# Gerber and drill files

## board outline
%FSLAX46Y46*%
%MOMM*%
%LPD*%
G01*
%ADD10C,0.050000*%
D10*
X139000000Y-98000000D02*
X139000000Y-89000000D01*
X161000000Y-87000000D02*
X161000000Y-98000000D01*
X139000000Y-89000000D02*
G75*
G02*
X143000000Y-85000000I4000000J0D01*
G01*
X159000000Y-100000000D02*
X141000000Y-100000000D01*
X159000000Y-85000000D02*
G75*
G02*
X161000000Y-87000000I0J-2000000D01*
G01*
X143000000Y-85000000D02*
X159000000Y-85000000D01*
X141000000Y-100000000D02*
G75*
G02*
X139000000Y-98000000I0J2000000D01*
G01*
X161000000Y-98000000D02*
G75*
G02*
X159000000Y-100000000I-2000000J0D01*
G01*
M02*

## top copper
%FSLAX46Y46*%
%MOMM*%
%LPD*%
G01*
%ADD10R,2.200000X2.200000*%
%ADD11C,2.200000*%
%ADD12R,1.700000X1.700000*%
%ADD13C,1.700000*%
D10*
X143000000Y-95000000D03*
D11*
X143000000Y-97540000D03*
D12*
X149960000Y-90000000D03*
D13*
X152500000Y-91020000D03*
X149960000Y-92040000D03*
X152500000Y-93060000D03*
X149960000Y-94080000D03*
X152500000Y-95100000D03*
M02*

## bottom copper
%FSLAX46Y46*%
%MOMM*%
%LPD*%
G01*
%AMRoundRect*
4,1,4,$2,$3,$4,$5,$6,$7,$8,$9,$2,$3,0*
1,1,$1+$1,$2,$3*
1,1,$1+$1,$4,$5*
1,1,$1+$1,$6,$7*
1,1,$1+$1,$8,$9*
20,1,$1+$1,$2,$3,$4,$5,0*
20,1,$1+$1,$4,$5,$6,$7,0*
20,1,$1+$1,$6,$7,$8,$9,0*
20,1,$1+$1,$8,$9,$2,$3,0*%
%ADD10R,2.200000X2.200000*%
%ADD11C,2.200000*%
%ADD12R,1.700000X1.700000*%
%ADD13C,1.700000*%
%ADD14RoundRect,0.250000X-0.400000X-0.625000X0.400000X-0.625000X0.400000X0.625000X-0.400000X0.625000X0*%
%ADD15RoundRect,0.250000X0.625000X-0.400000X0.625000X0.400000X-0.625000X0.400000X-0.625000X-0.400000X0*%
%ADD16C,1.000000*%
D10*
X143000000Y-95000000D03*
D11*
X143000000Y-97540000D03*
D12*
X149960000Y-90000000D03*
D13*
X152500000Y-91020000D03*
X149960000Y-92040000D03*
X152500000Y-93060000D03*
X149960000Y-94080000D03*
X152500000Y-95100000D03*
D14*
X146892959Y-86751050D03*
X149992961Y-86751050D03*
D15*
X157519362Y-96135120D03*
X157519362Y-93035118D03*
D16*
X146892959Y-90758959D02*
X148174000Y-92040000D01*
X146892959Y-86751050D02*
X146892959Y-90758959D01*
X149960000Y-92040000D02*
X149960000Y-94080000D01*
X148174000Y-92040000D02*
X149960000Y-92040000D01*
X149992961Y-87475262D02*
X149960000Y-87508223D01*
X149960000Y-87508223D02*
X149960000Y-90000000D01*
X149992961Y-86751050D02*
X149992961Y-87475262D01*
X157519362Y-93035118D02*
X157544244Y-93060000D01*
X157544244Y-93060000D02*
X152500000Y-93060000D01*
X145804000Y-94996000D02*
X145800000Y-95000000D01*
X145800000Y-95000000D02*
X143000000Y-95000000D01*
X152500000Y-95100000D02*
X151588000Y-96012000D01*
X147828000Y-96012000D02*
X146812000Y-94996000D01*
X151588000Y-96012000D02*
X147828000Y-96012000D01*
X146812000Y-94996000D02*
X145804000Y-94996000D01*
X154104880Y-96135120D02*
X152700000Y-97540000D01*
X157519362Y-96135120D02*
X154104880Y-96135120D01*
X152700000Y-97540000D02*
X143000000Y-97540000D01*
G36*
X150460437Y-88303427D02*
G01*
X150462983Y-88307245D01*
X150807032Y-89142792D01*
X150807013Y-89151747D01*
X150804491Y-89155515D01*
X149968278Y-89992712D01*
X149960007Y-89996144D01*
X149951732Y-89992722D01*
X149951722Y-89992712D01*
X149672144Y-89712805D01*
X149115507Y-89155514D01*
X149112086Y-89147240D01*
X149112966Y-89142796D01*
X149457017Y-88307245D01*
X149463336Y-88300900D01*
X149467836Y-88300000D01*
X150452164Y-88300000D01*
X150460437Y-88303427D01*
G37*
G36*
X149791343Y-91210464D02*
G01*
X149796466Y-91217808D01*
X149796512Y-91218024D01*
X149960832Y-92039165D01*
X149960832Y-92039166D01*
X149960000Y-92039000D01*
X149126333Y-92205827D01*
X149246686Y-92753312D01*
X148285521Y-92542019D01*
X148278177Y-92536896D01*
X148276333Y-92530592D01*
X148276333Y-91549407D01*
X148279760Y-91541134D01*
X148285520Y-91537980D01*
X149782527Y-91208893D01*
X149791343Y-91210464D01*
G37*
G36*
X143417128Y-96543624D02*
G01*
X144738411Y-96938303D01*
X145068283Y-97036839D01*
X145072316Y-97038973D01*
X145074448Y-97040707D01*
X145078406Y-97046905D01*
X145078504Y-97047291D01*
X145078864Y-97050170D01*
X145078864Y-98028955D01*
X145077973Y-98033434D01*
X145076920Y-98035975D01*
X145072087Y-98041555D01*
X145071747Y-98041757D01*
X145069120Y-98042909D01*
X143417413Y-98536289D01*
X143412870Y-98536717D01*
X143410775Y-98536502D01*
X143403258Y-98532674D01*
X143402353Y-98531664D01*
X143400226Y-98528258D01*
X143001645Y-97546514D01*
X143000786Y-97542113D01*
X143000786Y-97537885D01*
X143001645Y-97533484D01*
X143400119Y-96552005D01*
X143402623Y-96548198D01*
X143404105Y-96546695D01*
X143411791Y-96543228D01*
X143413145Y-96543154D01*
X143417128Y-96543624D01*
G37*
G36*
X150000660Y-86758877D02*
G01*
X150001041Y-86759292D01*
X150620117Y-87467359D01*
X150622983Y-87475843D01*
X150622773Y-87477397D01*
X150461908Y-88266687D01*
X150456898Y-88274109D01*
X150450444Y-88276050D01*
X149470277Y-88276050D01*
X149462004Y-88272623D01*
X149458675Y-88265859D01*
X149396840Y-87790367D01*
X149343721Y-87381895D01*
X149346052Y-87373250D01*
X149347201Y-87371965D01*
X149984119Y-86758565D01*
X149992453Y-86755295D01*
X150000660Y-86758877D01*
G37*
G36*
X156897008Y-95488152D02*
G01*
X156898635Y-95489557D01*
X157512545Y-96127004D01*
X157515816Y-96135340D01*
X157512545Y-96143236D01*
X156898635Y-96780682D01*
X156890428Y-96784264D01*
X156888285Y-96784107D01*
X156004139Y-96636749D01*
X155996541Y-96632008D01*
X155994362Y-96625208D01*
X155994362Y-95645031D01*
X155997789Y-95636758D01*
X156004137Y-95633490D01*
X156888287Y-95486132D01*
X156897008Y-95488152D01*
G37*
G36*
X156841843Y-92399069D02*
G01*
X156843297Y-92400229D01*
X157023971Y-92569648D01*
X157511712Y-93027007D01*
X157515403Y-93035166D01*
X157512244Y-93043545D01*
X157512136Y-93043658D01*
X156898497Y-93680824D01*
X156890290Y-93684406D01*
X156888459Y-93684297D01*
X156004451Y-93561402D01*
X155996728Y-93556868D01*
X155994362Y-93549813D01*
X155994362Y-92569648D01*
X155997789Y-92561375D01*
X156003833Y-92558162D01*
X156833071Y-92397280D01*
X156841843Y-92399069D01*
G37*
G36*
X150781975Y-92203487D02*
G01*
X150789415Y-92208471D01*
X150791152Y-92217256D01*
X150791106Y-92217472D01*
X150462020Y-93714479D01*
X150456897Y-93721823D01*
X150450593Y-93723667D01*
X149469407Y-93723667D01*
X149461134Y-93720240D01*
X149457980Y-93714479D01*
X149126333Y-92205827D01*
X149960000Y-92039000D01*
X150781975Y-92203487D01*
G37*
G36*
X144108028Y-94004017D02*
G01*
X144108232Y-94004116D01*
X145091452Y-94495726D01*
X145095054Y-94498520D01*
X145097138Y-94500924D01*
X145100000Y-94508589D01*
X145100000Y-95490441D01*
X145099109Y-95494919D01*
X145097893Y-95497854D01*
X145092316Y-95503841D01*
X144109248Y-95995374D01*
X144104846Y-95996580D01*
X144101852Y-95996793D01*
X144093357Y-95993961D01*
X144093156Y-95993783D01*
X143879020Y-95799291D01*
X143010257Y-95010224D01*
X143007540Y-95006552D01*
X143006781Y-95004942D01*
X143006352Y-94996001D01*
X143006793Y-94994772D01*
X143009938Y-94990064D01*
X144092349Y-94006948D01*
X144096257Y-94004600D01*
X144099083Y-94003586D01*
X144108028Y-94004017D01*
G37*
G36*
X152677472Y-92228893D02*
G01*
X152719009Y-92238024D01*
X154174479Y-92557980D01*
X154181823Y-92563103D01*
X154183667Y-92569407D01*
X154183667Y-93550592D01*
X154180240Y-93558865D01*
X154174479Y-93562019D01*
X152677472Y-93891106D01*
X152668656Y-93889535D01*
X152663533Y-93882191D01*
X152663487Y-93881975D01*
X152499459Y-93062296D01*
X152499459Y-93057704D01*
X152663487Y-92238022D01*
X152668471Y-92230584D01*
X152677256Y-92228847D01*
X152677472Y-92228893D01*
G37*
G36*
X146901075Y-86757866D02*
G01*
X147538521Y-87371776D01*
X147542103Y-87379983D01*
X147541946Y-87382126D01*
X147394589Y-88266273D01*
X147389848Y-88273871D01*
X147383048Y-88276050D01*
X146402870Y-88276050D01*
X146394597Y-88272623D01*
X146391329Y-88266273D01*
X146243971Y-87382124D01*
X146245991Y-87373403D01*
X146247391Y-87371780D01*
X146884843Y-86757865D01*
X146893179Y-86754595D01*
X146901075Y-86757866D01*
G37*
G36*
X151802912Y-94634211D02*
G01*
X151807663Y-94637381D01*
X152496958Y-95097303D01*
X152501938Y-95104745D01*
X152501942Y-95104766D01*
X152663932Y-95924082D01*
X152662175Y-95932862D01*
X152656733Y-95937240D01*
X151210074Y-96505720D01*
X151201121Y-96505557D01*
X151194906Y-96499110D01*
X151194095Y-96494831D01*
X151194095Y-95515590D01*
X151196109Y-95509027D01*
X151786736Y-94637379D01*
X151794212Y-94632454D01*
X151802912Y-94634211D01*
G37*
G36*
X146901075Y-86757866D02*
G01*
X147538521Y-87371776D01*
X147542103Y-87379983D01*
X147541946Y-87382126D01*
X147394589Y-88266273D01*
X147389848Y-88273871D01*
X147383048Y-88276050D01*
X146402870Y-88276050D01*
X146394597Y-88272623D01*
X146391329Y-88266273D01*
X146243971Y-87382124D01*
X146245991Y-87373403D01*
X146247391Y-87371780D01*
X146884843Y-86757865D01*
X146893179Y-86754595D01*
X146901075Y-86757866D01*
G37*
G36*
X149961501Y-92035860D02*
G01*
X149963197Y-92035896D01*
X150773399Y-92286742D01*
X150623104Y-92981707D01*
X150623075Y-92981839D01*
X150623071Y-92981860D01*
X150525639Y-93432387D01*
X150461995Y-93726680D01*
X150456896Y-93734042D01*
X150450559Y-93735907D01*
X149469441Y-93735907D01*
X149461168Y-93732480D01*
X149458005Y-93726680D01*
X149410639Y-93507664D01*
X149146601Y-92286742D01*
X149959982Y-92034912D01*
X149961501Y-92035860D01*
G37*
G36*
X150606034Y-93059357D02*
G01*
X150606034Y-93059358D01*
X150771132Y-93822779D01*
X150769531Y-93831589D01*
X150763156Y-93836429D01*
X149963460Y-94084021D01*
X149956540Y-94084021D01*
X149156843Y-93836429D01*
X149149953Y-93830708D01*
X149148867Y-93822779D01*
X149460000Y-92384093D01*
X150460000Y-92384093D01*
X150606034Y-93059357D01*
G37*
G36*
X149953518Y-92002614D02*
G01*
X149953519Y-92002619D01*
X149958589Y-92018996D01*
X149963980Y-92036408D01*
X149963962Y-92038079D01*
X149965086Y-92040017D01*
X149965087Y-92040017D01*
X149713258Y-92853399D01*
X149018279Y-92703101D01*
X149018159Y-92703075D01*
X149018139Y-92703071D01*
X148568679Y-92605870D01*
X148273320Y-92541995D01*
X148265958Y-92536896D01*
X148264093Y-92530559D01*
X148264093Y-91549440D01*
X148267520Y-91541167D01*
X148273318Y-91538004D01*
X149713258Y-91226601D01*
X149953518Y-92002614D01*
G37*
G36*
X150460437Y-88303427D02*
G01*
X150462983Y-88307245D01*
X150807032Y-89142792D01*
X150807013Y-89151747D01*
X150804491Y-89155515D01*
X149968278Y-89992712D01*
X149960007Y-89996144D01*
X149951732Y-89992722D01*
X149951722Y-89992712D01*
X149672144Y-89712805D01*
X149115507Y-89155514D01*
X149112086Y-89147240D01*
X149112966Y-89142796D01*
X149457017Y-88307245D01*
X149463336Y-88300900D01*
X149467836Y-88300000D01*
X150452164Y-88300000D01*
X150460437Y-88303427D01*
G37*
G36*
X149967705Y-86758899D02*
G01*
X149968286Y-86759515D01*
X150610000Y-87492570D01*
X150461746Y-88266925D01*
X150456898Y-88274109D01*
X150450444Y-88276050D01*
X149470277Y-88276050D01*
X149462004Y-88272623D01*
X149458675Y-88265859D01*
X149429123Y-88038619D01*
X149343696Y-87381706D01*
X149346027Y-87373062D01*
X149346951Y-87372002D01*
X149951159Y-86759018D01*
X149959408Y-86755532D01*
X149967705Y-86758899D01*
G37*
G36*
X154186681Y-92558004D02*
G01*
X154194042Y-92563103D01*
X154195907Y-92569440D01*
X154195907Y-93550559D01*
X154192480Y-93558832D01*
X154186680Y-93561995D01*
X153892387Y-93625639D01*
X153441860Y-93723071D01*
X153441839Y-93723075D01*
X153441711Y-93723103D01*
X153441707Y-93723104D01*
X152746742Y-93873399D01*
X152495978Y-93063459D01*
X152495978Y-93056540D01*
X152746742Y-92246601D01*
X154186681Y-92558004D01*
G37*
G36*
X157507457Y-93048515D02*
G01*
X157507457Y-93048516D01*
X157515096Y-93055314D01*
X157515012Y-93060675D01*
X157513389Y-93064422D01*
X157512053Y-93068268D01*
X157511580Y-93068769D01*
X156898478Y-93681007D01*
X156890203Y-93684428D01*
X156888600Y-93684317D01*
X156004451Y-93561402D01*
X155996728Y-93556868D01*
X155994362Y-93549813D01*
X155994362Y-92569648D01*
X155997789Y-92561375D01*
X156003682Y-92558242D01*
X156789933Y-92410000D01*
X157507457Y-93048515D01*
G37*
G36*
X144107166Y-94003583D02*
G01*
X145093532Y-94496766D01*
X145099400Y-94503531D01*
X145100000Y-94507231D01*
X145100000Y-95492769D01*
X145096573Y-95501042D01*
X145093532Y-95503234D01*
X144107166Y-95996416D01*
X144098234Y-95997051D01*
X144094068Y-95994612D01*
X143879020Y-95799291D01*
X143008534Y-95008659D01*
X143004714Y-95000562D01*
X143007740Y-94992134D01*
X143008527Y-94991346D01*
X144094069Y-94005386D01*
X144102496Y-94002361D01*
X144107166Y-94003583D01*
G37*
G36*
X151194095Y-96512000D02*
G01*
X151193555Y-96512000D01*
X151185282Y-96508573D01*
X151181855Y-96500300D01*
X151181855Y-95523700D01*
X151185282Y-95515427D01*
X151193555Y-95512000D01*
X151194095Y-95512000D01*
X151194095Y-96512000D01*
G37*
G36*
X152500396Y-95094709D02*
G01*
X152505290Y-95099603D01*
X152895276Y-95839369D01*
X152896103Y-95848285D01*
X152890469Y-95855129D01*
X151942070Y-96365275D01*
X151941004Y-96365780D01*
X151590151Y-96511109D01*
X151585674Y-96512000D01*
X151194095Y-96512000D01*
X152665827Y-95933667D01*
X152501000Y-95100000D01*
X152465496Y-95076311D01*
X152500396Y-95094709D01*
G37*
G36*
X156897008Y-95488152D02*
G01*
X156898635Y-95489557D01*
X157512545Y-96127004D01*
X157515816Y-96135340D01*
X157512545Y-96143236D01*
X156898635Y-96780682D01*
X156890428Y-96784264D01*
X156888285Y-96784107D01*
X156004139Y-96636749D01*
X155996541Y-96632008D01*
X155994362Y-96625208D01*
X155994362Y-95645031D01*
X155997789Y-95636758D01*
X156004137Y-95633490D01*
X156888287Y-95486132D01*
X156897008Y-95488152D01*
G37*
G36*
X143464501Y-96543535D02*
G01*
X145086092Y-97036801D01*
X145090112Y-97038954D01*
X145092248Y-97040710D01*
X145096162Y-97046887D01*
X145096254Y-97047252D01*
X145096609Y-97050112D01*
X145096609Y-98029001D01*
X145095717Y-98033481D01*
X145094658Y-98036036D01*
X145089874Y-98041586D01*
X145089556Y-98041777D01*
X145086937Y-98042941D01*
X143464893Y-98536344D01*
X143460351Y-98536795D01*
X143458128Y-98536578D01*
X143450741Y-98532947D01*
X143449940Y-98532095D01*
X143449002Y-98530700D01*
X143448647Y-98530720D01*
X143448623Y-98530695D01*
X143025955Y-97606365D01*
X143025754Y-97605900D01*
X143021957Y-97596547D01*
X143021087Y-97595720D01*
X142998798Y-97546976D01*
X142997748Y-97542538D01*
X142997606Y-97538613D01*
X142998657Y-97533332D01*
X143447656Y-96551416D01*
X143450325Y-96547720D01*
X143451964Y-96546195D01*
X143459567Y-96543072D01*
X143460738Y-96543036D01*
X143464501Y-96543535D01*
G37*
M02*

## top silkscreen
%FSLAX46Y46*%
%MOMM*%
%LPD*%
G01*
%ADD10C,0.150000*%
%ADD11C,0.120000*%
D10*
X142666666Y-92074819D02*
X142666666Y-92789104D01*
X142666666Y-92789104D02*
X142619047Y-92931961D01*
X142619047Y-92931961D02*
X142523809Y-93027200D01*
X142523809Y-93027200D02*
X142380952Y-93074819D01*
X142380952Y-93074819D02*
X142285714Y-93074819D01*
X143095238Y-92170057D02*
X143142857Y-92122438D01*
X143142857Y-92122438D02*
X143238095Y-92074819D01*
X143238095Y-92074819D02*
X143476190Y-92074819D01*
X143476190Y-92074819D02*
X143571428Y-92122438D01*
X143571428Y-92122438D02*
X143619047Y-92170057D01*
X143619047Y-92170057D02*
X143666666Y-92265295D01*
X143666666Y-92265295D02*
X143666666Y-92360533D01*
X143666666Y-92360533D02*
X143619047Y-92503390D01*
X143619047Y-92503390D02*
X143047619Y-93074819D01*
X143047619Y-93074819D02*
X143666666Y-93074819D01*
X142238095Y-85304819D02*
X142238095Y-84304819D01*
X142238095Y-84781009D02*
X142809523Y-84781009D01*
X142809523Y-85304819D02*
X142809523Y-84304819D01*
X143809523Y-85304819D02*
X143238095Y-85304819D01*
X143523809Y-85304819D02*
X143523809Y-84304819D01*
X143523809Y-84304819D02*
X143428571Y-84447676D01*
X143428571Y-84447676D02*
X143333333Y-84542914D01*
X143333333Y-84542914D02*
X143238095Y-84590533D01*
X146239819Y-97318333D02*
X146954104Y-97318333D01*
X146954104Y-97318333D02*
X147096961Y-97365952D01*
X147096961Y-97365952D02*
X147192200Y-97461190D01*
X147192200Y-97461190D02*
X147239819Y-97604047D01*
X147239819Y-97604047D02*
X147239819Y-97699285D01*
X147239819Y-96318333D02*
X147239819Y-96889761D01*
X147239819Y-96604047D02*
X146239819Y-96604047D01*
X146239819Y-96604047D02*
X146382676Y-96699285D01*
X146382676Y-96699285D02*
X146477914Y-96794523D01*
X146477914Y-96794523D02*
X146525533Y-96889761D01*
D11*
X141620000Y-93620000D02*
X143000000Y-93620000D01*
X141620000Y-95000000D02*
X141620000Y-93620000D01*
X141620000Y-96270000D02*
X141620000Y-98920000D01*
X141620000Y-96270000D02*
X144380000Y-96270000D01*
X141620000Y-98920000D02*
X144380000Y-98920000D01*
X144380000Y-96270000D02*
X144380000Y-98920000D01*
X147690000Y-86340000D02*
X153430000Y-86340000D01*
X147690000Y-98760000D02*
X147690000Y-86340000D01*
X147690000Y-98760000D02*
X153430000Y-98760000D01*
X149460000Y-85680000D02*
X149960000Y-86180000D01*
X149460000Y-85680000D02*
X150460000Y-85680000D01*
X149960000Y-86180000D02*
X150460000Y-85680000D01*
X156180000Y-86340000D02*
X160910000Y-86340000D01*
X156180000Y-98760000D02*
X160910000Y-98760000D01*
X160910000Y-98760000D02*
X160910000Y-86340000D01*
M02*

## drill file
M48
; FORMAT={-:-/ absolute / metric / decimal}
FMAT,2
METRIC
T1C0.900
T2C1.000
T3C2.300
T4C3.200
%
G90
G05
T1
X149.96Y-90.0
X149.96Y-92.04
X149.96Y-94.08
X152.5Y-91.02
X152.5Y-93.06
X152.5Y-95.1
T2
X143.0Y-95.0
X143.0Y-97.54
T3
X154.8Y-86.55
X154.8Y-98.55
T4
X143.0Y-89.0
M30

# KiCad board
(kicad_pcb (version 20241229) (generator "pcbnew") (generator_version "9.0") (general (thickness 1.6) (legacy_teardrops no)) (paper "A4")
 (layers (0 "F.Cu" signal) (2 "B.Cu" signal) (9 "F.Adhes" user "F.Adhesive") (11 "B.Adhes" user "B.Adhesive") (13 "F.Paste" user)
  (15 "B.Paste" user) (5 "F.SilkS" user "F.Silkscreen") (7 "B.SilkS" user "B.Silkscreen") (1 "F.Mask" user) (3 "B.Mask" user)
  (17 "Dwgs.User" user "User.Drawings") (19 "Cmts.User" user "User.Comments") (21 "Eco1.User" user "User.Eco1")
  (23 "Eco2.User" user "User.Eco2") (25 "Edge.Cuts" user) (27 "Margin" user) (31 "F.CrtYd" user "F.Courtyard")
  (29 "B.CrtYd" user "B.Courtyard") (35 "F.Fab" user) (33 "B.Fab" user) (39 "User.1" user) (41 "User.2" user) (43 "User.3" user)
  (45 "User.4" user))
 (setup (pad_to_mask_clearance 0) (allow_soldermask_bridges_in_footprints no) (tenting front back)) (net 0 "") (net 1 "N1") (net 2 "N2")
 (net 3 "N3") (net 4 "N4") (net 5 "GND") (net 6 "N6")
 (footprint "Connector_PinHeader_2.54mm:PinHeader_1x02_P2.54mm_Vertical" (layer "F.Cu") (at 143 95)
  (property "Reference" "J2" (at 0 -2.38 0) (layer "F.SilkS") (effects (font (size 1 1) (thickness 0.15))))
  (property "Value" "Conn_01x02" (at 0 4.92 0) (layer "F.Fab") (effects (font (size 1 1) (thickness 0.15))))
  (fp_line (start -1.38 -1.38) (end 0 -1.38) (stroke (width 0.12) (type solid)) (layer "F.SilkS"))
  (fp_line (start -1.38 0) (end -1.38 -1.38) (stroke (width 0.12) (type solid)) (layer "F.SilkS"))
  (fp_line (start -1.38 1.27) (end -1.38 3.92) (stroke (width 0.12) (type solid)) (layer "F.SilkS"))
  (fp_line (start -1.38 1.27) (end 1.38 1.27) (stroke (width 0.12) (type solid)) (layer "F.SilkS"))
  (fp_line (start -1.38 3.92) (end 1.38 3.92) (stroke (width 0.12) (type solid)) (layer "F.SilkS"))
  (fp_line (start 1.38 1.27) (end 1.38 3.92) (stroke (width 0.12) (type solid)) (layer "F.SilkS"))
  (pad "1" thru_hole rect (at 0 0) (size 2.2 2.2) (drill 1) (layers "*.Cu" "*.Mask") (remove_unused_layers no) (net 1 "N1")
   (teardrops (best_length_ratio 0.5) (max_length 1) (best_width_ratio 1) (max_width 2) (curved_edges no) (filter_ratio 0.9) (enabled yes)
    (allow_two_segments yes) (prefer_zone_connections yes)))
  (pad "2" thru_hole circle (at 0 2.54) (size 2.2 2.2) (drill 1) (layers "*.Cu" "*.Mask") (remove_unused_layers no) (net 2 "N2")
   (teardrops (best_length_ratio 0.5) (max_length 1) (best_width_ratio 1) (max_width 2) (curved_edges no) (filter_ratio 0.9) (enabled yes)
    (allow_two_segments yes) (prefer_zone_connections yes))))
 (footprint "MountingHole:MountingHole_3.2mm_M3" (layer "F.Cu") (at 143 89)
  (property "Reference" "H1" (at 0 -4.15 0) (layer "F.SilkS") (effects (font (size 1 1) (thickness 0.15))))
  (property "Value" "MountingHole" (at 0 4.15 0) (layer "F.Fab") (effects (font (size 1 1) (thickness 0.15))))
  (pad "" np_thru_hole circle (at 0 0) (size 3.2 3.2) (drill 3.2) (layers "*.Cu" "*.Mask")))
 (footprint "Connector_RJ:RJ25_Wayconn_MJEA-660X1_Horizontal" (layer "F.Cu") (at 149.96 90 90)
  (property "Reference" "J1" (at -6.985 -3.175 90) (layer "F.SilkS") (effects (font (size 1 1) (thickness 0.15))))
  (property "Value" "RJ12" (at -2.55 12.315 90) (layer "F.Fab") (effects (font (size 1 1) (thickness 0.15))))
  (fp_line (start 3.66 -2.27) (end 3.66 3.47) (stroke (width 0.12) (type solid)) (layer "F.SilkS"))
  (fp_line (start -8.76 -2.27) (end 3.66 -2.27) (stroke (width 0.12) (type solid)) (layer "F.SilkS"))
  (fp_line (start -8.76 -2.27) (end -8.76 3.47) (stroke (width 0.12) (type solid)) (layer "F.SilkS"))
  (fp_line (start 4.32 -0.5) (end 3.82 0) (stroke (width 0.12) (type solid)) (layer "F.SilkS"))
  (fp_line (start 4.32 -0.5) (end 4.32 0.5) (stroke (width 0.12) (type solid)) (layer "F.SilkS"))
  (fp_line (start 3.82 0) (end 4.32 0.5) (stroke (width 0.12) (type solid)) (layer "F.SilkS"))
  (fp_line (start 3.66 6.22) (end 3.66 10.95) (stroke (width 0.12) (type solid)) (layer "F.SilkS"))
  (fp_line (start -8.76 6.22) (end -8.76 10.95) (stroke (width 0.12) (type solid)) (layer "F.SilkS"))
  (fp_line (start -8.76 10.95) (end 3.66 10.95) (stroke (width 0.12) (type solid)) (layer "F.SilkS"))
  (pad "" np_thru_hole circle (at -8.55 4.84 90) (size 2.3 2.3) (drill 2.3) (layers "*.Cu" "*.Mask"))
  (pad "" np_thru_hole circle (at 3.45 4.84 90) (size 2.3 2.3) (drill 2.3) (layers "*.Cu" "*.Mask"))
  (pad "1" thru_hole rect (at 0 0 90) (size 1.7 1.7) (drill 0.9) (layers "*.Cu" "*.Mask") (remove_unused_layers no) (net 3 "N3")
   (teardrops (best_length_ratio 0.5) (max_length 1) (best_width_ratio 1) (max_width 2) (curved_edges no) (filter_ratio 0.9) (enabled yes)
    (allow_two_segments yes) (prefer_zone_connections yes)))
  (pad "2" thru_hole circle (at -1.02 2.54 90) (size 1.7 1.7) (drill 0.9) (layers "*.Cu" "*.Mask") (remove_unused_layers no) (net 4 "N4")
   (teardrops (best_length_ratio 0.5) (max_length 1) (best_width_ratio 1) (max_width 2) (curved_edges no) (filter_ratio 0.9) (enabled yes)
    (allow_two_segments yes) (prefer_zone_connections yes)))
  (pad "3" thru_hole circle (at -2.04 0 90) (size 1.7 1.7) (drill 0.9) (layers "*.Cu" "*.Mask") (remove_unused_layers no) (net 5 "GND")
   (teardrops (best_length_ratio 0.5) (max_length 1) (best_width_ratio 1) (max_width 2) (curved_edges no) (filter_ratio 0.9) (enabled yes)
    (allow_two_segments yes) (prefer_zone_connections yes)))
  (pad "4" thru_hole circle (at -3.06 2.54 90) (size 1.7 1.7) (drill 0.9) (layers "*.Cu" "*.Mask") (remove_unused_layers no) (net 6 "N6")
   (teardrops (best_length_ratio 0.5) (max_length 1) (best_width_ratio 1) (max_width 2) (curved_edges no) (filter_ratio 0.9) (enabled yes)
    (allow_two_segments yes) (prefer_zone_connections yes)))
  (pad "5" thru_hole circle (at -4.08 0 90) (size 1.7 1.7) (drill 0.9) (layers "*.Cu" "*.Mask") (remove_unused_layers no) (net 5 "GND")
   (teardrops (best_length_ratio 0.5) (max_length 1) (best_width_ratio 1) (max_width 2) (curved_edges no) (filter_ratio 0.9) (enabled yes)
    (allow_two_segments yes) (prefer_zone_connections yes)))
  (pad "6" thru_hole circle (at -5.1 2.54 90) (size 1.7 1.7) (drill 0.9) (layers "*.Cu" "*.Mask") (remove_unused_layers no) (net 1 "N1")
   (teardrops (best_length_ratio 0.5) (max_length 1) (best_width_ratio 1) (max_width 2) (curved_edges no) (filter_ratio 0.9) (enabled yes)
    (allow_two_segments yes) (prefer_zone_connections yes))))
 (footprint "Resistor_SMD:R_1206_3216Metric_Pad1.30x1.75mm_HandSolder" (layer "B.Cu") (at 148.44296 86.75105)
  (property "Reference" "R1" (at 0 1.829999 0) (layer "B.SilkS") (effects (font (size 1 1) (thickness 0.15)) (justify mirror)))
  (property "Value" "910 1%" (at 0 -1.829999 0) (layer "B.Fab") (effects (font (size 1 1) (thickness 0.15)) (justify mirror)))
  (pad "1" smd roundrect (at -1.550001 0) (size 1.3 1.75) (layers "B.Cu" "B.Mask" "B.Paste") (roundrect_rratio 0.192308) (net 5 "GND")
   (teardrops (best_length_ratio 0.5) (max_length 1) (best_width_ratio 1) (max_width 2) (curved_edges no) (filter_ratio 0.9) (enabled yes)
    (allow_two_segments yes) (prefer_zone_connections yes)))
  (pad "2" smd roundrect (at 1.550001 0) (size 1.3 1.75) (layers "B.Cu" "B.Mask" "B.Paste") (roundrect_rratio 0.192308) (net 3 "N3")
   (teardrops (best_length_ratio 0.5) (max_length 1) (best_width_ratio 1) (max_width 2) (curved_edges no) (filter_ratio 0.9) (enabled yes)
    (allow_two_segments yes) (prefer_zone_connections yes))))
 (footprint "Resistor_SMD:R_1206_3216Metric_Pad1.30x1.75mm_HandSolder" (layer "B.Cu") (at 157.519362 94.585119 90)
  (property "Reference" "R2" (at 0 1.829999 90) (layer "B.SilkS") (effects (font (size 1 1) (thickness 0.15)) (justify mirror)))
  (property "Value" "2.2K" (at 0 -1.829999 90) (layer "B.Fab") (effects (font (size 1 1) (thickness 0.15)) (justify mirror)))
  (pad "1" smd roundrect (at -1.550001 0 90) (size 1.3 1.75) (layers "B.Cu" "B.Mask" "B.Paste") (roundrect_rratio 0.192308) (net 2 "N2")
   (teardrops (best_length_ratio 0.5) (max_length 1) (best_width_ratio 1) (max_width 2) (curved_edges no) (filter_ratio 0.9) (enabled yes)
    (allow_two_segments yes) (prefer_zone_connections yes)))
  (pad "2" smd roundrect (at 1.550001 0 90) (size 1.3 1.75) (layers "B.Cu" "B.Mask" "B.Paste") (roundrect_rratio 0.192308) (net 6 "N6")
   (teardrops (best_length_ratio 0.5) (max_length 1) (best_width_ratio 1) (max_width 2) (curved_edges no) (filter_ratio 0.9) (enabled yes)
    (allow_two_segments yes) (prefer_zone_connections yes))))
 (gr_line (start 139 98) (end 139 89) (stroke (width 0.05) (type default)) (layer "Edge.Cuts"))
 (gr_line (start 161 87) (end 161 98) (stroke (width 0.05) (type default)) (layer "Edge.Cuts"))
 (gr_arc (start 139 89) (mid 140.171573 86.171573) (end 143 85) (stroke (width 0.05) (type default)) (layer "Edge.Cuts"))
 (gr_line (start 159 100) (end 141 100) (stroke (width 0.05) (type default)) (layer "Edge.Cuts"))
 (gr_arc (start 159 85) (mid 160.414214 85.585786) (end 161 87) (stroke (width 0.05) (type default)) (layer "Edge.Cuts"))
 (gr_line (start 143 85) (end 159 85) (stroke (width 0.05) (type default)) (layer "Edge.Cuts"))
 (gr_arc (start 141 100) (mid 139.585786 99.414214) (end 139 98) (stroke (width 0.05) (type default)) (layer "Edge.Cuts"))
 (gr_arc (start 161 98) (mid 160.414214 99.414214) (end 159 100) (stroke (width 0.05) (type default)) (layer "Edge.Cuts"))
 (segment (start 146.892959 90.758959) (end 148.174 92.04) (width 1) (layer "B.Cu") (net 5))
 (segment (start 146.892959 86.75105) (end 146.892959 90.758959) (width 1) (layer "B.Cu") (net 5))
 (segment (start 149.96 92.04) (end 149.96 94.08) (width 1) (layer "B.Cu") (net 5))
 (segment (start 148.174 92.04) (end 149.96 92.04) (width 1) (layer "B.Cu") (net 5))
 (segment (start 149.992961 87.475262) (end 149.96 87.508223) (width 1) (layer "B.Cu") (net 3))
 (segment (start 149.96 87.508223) (end 149.96 90) (width 1) (layer "B.Cu") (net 3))
 (segment (start 149.992961 86.75105) (end 149.992961 87.475262) (width 1) (layer "B.Cu") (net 3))
 (segment (start 157.519362 93.035118) (end 157.544244 93.06) (width 1) (layer "B.Cu") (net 6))
 (segment (start 157.544244 93.06) (end 152.5 93.06) (width 1) (layer "B.Cu") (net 6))
 (segment (start 145.804 94.996) (end 145.8 95) (width 1) (layer "B.Cu") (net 1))
 (segment (start 145.8 95) (end 143 95) (width 1) (layer "B.Cu") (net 1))
 (segment (start 152.5 95.1) (end 151.588 96.012) (width 1) (layer "B.Cu") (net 1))
 (segment (start 147.828 96.012) (end 146.812 94.996) (width 1) (layer "B.Cu") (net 1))
 (segment (start 151.588 96.012) (end 147.828 96.012) (width 1) (layer "B.Cu") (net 1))
 (segment (start 146.812 94.996) (end 145.804 94.996) (width 1) (layer "B.Cu") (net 1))
 (segment (start 154.10488 96.13512) (end 152.7 97.54) (width 1) (layer "B.Cu") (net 2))
 (segment (start 157.519362 96.13512) (end 154.10488 96.13512) (width 1) (layer "B.Cu") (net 2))
 (segment (start 152.7 97.54) (end 143 97.54) (width 1) (layer "B.Cu") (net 2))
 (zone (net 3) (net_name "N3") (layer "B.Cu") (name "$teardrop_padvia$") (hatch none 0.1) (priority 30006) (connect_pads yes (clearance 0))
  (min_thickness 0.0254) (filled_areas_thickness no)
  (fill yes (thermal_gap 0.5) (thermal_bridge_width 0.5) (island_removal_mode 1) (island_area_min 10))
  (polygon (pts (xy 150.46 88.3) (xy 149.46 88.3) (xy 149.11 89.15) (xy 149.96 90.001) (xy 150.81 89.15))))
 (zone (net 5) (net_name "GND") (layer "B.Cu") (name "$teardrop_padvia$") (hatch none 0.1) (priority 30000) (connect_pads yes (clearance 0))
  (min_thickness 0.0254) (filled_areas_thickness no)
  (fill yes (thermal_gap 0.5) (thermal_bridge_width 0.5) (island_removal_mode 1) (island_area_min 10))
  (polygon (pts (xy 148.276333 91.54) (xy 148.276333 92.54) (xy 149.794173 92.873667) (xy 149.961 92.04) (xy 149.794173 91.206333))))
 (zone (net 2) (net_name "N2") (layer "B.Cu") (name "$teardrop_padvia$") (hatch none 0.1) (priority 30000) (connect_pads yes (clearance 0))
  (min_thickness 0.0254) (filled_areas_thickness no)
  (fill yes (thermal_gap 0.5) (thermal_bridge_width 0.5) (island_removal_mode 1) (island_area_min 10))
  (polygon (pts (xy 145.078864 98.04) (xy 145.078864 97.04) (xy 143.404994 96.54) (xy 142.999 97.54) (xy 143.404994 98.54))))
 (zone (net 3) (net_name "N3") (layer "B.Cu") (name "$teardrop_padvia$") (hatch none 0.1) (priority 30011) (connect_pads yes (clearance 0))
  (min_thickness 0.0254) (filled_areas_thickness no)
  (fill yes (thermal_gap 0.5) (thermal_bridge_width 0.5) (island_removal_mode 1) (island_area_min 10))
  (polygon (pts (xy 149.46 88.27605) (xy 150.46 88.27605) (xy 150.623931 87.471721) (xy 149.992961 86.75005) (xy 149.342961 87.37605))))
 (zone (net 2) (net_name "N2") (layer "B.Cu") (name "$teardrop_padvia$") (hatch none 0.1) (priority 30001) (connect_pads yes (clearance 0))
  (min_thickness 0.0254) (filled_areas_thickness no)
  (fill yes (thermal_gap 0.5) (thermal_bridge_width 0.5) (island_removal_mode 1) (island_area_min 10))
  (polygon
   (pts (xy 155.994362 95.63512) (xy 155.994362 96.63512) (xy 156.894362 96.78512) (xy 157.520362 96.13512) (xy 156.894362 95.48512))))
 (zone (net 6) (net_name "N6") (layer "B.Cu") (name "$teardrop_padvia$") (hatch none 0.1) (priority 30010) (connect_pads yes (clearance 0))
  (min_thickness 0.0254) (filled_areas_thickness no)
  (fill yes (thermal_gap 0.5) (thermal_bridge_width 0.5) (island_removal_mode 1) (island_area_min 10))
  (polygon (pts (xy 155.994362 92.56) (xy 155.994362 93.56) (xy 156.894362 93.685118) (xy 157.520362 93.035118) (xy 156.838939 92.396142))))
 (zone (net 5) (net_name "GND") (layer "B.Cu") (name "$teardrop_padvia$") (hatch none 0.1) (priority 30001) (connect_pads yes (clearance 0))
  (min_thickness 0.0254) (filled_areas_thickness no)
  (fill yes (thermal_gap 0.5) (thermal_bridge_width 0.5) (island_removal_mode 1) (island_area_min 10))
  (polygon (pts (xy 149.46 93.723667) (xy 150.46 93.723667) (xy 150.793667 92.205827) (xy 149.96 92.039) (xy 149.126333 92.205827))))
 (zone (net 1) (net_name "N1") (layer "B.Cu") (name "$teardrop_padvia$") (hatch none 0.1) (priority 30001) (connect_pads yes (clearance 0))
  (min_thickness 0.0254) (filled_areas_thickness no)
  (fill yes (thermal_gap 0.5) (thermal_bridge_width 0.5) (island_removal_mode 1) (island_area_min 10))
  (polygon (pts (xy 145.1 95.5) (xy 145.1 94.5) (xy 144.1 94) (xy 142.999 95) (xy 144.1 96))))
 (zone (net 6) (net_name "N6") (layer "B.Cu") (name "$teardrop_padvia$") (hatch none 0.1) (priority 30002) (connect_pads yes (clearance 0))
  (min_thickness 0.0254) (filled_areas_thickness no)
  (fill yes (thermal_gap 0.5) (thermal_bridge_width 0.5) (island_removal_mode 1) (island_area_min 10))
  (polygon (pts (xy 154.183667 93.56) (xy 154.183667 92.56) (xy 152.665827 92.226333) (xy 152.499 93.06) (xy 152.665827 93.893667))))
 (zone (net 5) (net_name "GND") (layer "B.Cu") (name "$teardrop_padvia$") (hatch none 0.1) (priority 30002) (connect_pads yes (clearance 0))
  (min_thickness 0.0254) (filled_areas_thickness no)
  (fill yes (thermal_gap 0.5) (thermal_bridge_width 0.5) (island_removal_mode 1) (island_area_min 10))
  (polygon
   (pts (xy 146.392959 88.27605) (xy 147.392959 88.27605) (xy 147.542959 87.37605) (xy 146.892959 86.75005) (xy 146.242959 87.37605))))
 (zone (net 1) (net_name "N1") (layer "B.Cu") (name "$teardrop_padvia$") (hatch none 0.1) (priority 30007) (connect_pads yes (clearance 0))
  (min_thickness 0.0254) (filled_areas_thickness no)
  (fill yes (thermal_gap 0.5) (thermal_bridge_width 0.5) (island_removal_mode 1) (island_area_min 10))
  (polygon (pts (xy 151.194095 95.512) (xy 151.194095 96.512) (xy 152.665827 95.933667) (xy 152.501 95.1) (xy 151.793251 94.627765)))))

